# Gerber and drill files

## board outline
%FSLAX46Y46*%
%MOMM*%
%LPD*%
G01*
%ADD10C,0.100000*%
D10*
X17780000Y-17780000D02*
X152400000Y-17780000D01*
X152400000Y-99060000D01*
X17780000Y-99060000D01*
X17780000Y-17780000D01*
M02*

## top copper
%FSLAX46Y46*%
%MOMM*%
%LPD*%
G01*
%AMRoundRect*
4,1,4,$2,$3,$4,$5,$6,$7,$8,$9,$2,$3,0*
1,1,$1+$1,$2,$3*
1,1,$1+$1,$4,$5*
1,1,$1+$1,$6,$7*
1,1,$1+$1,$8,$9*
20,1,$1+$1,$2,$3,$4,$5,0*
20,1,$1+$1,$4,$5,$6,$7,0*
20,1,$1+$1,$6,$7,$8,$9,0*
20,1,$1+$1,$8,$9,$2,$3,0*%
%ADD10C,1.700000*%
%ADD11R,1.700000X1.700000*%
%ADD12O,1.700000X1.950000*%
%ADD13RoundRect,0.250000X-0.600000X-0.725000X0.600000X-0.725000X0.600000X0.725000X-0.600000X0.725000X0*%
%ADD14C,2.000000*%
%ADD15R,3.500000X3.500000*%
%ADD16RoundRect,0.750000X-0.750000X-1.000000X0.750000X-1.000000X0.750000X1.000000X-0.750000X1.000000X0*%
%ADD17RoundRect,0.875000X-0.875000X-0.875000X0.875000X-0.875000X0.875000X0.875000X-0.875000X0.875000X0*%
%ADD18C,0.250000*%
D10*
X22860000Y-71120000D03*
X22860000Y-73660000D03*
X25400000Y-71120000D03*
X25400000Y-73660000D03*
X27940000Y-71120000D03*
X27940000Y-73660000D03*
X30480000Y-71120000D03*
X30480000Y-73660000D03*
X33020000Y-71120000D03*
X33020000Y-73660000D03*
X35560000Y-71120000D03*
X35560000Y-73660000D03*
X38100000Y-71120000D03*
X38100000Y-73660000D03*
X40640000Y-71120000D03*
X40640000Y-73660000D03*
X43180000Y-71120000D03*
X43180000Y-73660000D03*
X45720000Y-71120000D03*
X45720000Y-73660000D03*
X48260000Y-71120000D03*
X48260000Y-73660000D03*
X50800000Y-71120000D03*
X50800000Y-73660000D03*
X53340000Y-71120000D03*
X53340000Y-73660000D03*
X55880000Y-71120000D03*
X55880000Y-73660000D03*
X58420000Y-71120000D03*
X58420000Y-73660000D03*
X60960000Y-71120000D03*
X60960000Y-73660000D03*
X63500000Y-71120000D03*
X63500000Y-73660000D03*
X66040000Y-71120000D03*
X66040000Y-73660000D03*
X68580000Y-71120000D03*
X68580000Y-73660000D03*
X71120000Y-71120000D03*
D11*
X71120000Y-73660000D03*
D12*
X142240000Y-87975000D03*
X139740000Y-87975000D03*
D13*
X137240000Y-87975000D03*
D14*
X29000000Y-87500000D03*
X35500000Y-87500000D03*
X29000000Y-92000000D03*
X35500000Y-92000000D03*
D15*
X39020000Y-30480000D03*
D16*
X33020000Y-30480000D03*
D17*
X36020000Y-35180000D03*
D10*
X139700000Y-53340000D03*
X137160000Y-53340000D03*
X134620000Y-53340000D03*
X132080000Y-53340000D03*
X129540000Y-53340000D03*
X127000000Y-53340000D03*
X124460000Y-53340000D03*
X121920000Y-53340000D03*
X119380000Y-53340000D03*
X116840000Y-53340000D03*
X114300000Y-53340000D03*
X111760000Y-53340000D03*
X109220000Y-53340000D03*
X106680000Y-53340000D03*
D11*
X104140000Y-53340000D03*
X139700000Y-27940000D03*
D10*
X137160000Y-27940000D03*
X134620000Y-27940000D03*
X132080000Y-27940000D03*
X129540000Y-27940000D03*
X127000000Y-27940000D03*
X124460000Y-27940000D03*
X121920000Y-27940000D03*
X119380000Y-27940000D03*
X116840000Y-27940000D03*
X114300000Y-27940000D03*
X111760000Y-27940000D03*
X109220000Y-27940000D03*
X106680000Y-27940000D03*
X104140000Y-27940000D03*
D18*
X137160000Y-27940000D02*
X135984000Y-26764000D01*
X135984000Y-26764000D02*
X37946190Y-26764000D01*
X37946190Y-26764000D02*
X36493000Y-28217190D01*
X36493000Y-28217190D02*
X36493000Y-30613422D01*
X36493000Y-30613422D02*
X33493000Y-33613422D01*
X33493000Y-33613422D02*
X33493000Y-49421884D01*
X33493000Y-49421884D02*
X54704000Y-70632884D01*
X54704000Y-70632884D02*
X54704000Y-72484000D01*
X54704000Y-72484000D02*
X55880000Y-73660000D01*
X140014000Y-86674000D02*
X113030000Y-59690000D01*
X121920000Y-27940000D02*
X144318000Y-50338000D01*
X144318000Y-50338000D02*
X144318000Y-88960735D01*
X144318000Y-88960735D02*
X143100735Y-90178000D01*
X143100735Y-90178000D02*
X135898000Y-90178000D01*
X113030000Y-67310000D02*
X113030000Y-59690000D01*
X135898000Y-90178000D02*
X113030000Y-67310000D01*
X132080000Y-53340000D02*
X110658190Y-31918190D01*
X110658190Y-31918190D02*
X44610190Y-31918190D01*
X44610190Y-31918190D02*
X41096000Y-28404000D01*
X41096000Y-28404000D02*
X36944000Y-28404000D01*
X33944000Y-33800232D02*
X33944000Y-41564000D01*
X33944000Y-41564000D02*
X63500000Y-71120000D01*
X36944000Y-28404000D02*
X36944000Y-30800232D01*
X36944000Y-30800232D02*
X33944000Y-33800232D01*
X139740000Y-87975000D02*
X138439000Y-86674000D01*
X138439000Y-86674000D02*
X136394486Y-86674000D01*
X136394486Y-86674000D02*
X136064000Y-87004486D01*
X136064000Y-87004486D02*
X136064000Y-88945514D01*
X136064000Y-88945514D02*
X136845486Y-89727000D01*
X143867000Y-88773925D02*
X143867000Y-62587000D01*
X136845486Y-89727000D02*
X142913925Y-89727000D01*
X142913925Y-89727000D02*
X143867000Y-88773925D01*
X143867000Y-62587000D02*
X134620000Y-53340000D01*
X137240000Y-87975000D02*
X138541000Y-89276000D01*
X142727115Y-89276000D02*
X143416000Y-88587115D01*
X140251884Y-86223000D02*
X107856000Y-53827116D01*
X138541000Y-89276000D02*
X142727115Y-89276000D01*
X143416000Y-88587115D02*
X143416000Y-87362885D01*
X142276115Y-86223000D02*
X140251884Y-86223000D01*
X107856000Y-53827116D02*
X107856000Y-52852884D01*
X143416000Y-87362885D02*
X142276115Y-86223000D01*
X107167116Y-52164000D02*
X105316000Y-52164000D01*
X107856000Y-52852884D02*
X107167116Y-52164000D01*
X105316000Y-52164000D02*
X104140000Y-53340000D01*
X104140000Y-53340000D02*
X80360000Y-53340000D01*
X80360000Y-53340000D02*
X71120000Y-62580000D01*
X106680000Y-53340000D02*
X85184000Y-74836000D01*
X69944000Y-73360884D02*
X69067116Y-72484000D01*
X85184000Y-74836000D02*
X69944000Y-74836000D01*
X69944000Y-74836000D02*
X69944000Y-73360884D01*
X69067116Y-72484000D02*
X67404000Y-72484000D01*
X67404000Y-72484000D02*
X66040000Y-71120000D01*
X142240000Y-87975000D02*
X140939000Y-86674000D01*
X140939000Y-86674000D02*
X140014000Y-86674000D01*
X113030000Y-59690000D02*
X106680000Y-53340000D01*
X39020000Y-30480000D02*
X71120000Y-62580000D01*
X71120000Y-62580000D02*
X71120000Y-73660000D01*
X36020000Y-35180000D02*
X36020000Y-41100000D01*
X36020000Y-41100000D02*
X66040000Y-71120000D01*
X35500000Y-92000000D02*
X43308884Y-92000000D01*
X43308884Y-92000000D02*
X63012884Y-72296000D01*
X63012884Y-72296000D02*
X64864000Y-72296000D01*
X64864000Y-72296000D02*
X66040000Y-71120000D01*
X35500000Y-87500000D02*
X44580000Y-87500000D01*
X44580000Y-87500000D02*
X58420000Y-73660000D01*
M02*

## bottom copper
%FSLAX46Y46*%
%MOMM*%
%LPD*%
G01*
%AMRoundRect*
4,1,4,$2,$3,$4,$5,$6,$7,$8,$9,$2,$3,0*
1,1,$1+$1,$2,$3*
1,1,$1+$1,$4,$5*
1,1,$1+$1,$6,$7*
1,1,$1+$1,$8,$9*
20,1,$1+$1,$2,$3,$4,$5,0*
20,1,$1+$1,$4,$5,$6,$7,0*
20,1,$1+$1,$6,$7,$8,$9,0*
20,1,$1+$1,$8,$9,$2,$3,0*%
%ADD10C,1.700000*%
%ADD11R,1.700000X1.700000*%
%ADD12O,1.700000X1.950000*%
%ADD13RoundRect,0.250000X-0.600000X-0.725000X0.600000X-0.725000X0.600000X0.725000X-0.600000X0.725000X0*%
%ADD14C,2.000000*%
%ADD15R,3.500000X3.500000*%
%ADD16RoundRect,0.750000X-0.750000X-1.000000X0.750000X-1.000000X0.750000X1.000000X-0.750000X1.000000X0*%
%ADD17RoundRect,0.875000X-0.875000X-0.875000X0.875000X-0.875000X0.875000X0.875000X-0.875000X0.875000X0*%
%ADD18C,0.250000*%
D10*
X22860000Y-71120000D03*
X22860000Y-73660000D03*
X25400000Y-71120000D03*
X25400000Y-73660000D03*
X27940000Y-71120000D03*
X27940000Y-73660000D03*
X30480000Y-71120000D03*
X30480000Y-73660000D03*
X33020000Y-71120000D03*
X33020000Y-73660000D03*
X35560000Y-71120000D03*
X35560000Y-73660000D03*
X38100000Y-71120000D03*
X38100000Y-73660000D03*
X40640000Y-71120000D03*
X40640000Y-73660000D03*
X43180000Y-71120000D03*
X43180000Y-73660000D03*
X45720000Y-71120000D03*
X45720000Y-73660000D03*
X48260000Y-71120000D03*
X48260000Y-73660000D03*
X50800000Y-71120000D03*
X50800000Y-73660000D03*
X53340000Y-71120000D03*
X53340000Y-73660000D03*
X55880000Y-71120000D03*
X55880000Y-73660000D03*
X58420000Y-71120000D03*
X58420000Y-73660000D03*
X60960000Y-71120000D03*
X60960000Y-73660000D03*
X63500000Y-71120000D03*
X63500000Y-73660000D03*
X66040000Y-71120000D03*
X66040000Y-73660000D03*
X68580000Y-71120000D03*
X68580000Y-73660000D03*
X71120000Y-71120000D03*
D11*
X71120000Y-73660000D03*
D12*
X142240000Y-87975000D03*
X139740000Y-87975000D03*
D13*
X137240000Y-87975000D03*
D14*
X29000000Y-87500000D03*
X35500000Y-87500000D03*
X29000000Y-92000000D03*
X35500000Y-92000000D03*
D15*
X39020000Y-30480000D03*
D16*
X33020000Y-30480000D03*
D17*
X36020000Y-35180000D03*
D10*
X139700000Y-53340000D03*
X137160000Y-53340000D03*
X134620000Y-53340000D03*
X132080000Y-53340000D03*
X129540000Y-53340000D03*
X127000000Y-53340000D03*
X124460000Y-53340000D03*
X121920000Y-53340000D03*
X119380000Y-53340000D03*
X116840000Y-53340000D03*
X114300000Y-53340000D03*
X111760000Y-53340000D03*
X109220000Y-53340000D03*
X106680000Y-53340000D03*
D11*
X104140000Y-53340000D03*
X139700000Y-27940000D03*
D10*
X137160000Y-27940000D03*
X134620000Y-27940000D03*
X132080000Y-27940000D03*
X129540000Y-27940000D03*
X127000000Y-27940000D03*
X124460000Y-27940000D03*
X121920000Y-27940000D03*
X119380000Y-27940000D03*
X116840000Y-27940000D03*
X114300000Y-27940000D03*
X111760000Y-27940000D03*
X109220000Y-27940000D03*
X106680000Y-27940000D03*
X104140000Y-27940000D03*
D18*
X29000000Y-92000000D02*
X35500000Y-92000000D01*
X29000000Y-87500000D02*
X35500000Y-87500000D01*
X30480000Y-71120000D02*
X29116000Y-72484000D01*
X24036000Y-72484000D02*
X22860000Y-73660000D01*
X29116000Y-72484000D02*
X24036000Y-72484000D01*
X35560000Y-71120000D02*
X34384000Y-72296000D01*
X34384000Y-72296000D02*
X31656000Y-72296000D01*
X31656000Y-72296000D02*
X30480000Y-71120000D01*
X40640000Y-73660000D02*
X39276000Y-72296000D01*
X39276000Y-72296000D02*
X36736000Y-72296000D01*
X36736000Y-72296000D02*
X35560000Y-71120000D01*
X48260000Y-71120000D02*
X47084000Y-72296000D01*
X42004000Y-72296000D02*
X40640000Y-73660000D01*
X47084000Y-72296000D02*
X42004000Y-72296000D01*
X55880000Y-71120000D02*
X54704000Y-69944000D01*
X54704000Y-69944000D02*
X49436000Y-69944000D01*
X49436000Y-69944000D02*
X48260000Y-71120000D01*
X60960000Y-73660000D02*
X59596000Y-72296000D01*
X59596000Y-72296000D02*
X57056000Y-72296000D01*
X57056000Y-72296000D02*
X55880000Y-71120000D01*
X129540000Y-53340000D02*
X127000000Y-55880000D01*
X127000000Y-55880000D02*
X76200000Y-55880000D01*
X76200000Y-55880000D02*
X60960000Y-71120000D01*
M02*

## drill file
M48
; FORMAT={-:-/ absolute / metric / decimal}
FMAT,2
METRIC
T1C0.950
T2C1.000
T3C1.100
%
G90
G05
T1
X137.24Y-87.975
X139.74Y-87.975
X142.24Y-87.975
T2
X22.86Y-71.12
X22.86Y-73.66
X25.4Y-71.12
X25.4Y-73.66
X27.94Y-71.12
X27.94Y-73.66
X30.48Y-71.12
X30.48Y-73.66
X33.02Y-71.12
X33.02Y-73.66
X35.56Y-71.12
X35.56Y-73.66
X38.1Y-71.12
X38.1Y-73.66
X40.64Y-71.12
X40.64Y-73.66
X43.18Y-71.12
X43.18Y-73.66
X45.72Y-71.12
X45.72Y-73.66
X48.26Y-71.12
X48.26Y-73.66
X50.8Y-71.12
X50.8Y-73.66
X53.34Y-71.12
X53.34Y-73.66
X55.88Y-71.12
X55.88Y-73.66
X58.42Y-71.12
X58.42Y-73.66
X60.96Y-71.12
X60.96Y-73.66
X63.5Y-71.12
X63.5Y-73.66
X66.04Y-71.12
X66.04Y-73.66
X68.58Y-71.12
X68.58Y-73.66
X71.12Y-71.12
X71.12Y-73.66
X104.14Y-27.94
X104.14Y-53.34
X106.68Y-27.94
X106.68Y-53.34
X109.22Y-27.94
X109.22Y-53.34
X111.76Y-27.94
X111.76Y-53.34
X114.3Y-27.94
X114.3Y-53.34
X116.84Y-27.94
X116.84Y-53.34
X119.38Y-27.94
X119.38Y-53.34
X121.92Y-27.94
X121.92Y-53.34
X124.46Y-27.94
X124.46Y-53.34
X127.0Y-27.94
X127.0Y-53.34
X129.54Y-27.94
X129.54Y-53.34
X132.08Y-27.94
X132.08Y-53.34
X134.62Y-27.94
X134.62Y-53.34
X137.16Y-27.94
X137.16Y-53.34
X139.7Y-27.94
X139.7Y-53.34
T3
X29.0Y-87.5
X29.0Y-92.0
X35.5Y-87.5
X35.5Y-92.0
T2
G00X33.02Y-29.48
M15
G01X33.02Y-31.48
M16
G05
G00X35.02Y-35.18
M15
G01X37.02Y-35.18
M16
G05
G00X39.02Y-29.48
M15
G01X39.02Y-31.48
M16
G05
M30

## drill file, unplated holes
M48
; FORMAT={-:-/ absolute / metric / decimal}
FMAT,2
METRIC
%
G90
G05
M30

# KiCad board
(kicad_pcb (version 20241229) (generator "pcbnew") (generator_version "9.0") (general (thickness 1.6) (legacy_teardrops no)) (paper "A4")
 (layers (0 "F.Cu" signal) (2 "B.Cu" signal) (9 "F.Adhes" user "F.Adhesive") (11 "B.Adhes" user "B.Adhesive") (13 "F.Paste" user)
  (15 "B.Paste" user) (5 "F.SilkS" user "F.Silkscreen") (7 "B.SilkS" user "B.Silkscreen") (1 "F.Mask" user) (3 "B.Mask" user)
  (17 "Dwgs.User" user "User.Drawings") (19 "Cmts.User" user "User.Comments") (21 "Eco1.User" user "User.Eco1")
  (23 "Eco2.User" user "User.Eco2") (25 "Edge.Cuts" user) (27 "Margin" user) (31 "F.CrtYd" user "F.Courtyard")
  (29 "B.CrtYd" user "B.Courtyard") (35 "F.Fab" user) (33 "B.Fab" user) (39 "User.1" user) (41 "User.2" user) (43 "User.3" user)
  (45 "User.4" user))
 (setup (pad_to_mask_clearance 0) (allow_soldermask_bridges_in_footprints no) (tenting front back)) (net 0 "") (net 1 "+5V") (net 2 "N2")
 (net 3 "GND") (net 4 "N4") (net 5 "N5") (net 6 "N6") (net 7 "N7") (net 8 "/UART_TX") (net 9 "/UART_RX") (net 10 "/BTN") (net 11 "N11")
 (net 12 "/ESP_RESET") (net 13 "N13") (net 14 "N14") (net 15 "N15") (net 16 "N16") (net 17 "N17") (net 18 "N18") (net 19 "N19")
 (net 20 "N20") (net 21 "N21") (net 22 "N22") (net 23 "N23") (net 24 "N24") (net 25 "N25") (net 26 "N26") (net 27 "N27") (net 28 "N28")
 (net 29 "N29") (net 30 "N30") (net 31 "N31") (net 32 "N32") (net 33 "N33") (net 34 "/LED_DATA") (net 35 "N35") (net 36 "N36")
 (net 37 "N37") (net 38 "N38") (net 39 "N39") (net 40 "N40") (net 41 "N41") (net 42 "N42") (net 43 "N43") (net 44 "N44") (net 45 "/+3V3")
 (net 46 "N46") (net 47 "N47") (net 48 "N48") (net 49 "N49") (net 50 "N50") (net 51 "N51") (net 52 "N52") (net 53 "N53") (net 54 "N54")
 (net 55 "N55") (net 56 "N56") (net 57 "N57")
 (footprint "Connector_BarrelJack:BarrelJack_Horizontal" (layer "F.Cu") (at 39.02 30.48)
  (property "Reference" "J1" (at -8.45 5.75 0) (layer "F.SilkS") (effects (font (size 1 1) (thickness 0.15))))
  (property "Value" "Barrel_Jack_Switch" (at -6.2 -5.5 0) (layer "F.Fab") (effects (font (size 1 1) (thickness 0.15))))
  (pad "1" thru_hole rect (at 0 0) (size 3.5 3.5) (drill oval 1 3) (layers "*.Cu" "*.Mask") (remove_unused_layers no) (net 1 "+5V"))
  (pad "2" thru_hole roundrect (at -6 0) (size 3 3.5) (drill oval 1 3) (layers "*.Cu" "*.Mask") (remove_unused_layers no)
   (roundrect_rratio 0.25) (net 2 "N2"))
  (pad "3" thru_hole roundrect (at -3 4.7) (size 3.5 3.5) (drill oval 3 1) (layers "*.Cu" "*.Mask") (remove_unused_layers no)
   (roundrect_rratio 0.25) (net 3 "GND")))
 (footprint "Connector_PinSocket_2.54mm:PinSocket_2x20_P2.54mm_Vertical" (layer "F.Cu") (at 71.12 73.66 -90)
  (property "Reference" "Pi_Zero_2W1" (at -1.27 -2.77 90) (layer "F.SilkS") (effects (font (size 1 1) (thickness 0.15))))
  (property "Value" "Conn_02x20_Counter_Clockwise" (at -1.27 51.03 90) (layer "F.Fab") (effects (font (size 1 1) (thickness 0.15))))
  (pad "1" thru_hole rect (at 0 0 270) (size 1.7 1.7) (drill 1) (layers "*.Cu" "*.Mask") (remove_unused_layers no) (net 1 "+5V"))
  (pad "2" thru_hole circle (at -2.54 0 270) (size 1.7 1.7) (drill 1) (layers "*.Cu" "*.Mask") (remove_unused_layers no) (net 1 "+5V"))
  (pad "3" thru_hole circle (at 0 2.54 270) (size 1.7 1.7) (drill 1) (layers "*.Cu" "*.Mask") (remove_unused_layers no) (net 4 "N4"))
  (pad "4" thru_hole circle (at -2.54 2.54 270) (size 1.7 1.7) (drill 1) (layers "*.Cu" "*.Mask") (remove_unused_layers no) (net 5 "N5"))
  (pad "5" thru_hole circle (at 0 5.08 270) (size 1.7 1.7) (drill 1) (layers "*.Cu" "*.Mask") (remove_unused_layers no) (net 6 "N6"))
  (pad "6" thru_hole circle (at -2.54 5.08 270) (size 1.7 1.7) (drill 1) (layers "*.Cu" "*.Mask") (remove_unused_layers no) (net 3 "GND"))
  (pad "7" thru_hole circle (at 0 7.62 270) (size 1.7 1.7) (drill 1) (layers "*.Cu" "*.Mask") (remove_unused_layers no) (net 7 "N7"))
  (pad "8" thru_hole circle (at -2.54 7.62 270) (size 1.7 1.7) (drill 1) (layers "*.Cu" "*.Mask") (remove_unused_layers no)
   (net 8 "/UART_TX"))
  (pad "9" thru_hole circle (at 0 10.16 270) (size 1.7 1.7) (drill 1) (layers "*.Cu" "*.Mask") (remove_unused_layers no) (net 3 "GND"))
  (pad "10" thru_hole circle (at -2.54 10.16 270) (size 1.7 1.7) (drill 1) (layers "*.Cu" "*.Mask") (remove_unused_layers no)
   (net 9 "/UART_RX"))
  (pad "11" thru_hole circle (at 0 12.7 270) (size 1.7 1.7) (drill 1) (layers "*.Cu" "*.Mask") (remove_unused_layers no) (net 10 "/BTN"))
  (pad "12" thru_hole circle (at -2.54 12.7 270) (size 1.7 1.7) (drill 1) (layers "*.Cu" "*.Mask") (remove_unused_layers no) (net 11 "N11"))
  (pad "13" thru_hole circle (at 0 15.24 270) (size 1.7 1.7) (drill 1) (layers "*.Cu" "*.Mask") (remove_unused_layers no)
   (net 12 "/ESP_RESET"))
  (pad "14" thru_hole circle (at -2.54 15.24 270) (size 1.7 1.7) (drill 1) (layers "*.Cu" "*.Mask") (remove_unused_layers no) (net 3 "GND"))
  (pad "15" thru_hole circle (at 0 17.78 270) (size 1.7 1.7) (drill 1) (layers "*.Cu" "*.Mask") (remove_unused_layers no) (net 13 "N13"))
  (pad "16" thru_hole circle (at -2.54 17.78 270) (size 1.7 1.7) (drill 1) (layers "*.Cu" "*.Mask") (remove_unused_layers no) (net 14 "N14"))
  (pad "17" thru_hole circle (at 0 20.32 270) (size 1.7 1.7) (drill 1) (layers "*.Cu" "*.Mask") (remove_unused_layers no) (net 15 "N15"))
  (pad "18" thru_hole circle (at -2.54 20.32 270) (size 1.7 1.7) (drill 1) (layers "*.Cu" "*.Mask") (remove_unused_layers no) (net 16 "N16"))
  (pad "19" thru_hole circle (at 0 22.86 270) (size 1.7 1.7) (drill 1) (layers "*.Cu" "*.Mask") (remove_unused_layers no) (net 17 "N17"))
  (pad "20" thru_hole circle (at -2.54 22.86 270) (size 1.7 1.7) (drill 1) (layers "*.Cu" "*.Mask") (remove_unused_layers no) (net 3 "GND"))
  (pad "21" thru_hole circle (at 0 25.4 270) (size 1.7 1.7) (drill 1) (layers "*.Cu" "*.Mask") (remove_unused_layers no) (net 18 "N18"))
  (pad "22" thru_hole circle (at -2.54 25.4 270) (size 1.7 1.7) (drill 1) (layers "*.Cu" "*.Mask") (remove_unused_layers no) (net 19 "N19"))
  (pad "23" thru_hole circle (at 0 27.94 270) (size 1.7 1.7) (drill 1) (layers "*.Cu" "*.Mask") (remove_unused_layers no) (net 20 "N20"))
  (pad "24" thru_hole circle (at -2.54 27.94 270) (size 1.7 1.7) (drill 1) (layers "*.Cu" "*.Mask") (remove_unused_layers no) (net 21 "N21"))
  (pad "25" thru_hole circle (at 0 30.48 270) (size 1.7 1.7) (drill 1) (layers "*.Cu" "*.Mask") (remove_unused_layers no) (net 3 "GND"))
  (pad "26" thru_hole circle (at -2.54 30.48 270) (size 1.7 1.7) (drill 1) (layers "*.Cu" "*.Mask") (remove_unused_layers no) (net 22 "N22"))
  (pad "27" thru_hole circle (at 0 33.02 270) (size 1.7 1.7) (drill 1) (layers "*.Cu" "*.Mask") (remove_unused_layers no) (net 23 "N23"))
  (pad "28" thru_hole circle (at -2.54 33.02 270) (size 1.7 1.7) (drill 1) (layers "*.Cu" "*.Mask") (remove_unused_layers no) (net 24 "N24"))
  (pad "29" thru_hole circle (at 0 35.56 270) (size 1.7 1.7) (drill 1) (layers "*.Cu" "*.Mask") (remove_unused_layers no) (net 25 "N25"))
  (pad "30" thru_hole circle (at -2.54 35.56 270) (size 1.7 1.7) (drill 1) (layers "*.Cu" "*.Mask") (remove_unused_layers no) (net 3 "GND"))
  (pad "31" thru_hole circle (at 0 38.1 270) (size 1.7 1.7) (drill 1) (layers "*.Cu" "*.Mask") (remove_unused_layers no) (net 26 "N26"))
  (pad "32" thru_hole circle (at -2.54 38.1 270) (size 1.7 1.7) (drill 1) (layers "*.Cu" "*.Mask") (remove_unused_layers no) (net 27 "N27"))
  (pad "33" thru_hole circle (at 0 40.64 270) (size 1.7 1.7) (drill 1) (layers "*.Cu" "*.Mask") (remove_unused_layers no) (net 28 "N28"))
  (pad "34" thru_hole circle (at -2.54 40.64 270) (size 1.7 1.7) (drill 1) (layers "*.Cu" "*.Mask") (remove_unused_layers no) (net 3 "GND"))
  (pad "35" thru_hole circle (at 0 43.18 270) (size 1.7 1.7) (drill 1) (layers "*.Cu" "*.Mask") (remove_unused_layers no) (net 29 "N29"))
  (pad "36" thru_hole circle (at -2.54 43.18 270) (size 1.7 1.7) (drill 1) (layers "*.Cu" "*.Mask") (remove_unused_layers no) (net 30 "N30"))
  (pad "37" thru_hole circle (at 0 45.72 270) (size 1.7 1.7) (drill 1) (layers "*.Cu" "*.Mask") (remove_unused_layers no) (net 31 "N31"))
  (pad "38" thru_hole circle (at -2.54 45.72 270) (size 1.7 1.7) (drill 1) (layers "*.Cu" "*.Mask") (remove_unused_layers no) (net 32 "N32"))
  (pad "39" thru_hole circle (at 0 48.26 270) (size 1.7 1.7) (drill 1) (layers "*.Cu" "*.Mask") (remove_unused_layers no) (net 3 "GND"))
  (pad "40" thru_hole circle (at -2.54 48.26 270) (size 1.7 1.7) (drill 1) (layers "*.Cu" "*.Mask") (remove_unused_layers no) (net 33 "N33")))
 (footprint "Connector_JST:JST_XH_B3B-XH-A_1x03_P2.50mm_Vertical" (layer "F.Cu") (at 137.24 87.975)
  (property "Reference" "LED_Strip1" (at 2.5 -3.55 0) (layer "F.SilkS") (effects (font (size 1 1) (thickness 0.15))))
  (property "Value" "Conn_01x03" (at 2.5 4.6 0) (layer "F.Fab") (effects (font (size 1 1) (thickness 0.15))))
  (pad "1" thru_hole roundrect (at 0 0) (size 1.7 1.95) (drill 0.95) (layers "*.Cu" "*.Mask") (remove_unused_layers no)
   (roundrect_rratio 0.147059) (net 1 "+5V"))
  (pad "2" thru_hole oval (at 2.5 0) (size 1.7 1.95) (drill 0.95) (layers "*.Cu" "*.Mask") (remove_unused_layers no) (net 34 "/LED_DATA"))
  (pad "3" thru_hole oval (at 5 0) (size 1.7 1.95) (drill 0.95) (layers "*.Cu" "*.Mask") (remove_unused_layers no) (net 3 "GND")))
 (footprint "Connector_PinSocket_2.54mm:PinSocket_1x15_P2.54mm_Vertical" (layer "F.Cu") (at 104.14 53.34 90)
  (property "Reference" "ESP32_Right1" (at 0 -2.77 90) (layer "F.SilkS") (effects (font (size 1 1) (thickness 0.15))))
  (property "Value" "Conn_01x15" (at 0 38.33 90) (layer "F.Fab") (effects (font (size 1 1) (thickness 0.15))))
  (pad "1" thru_hole rect (at 0 0 90) (size 1.7 1.7) (drill 1) (layers "*.Cu" "*.Mask") (remove_unused_layers no) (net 1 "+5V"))
  (pad "2" thru_hole circle (at 0 2.54 90) (size 1.7 1.7) (drill 1) (layers "*.Cu" "*.Mask") (remove_unused_layers no) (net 3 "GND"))
  (pad "3" thru_hole circle (at 0 5.08 90) (size 1.7 1.7) (drill 1) (layers "*.Cu" "*.Mask") (remove_unused_layers no) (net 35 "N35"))
  (pad "4" thru_hole circle (at 0 7.62 90) (size 1.7 1.7) (drill 1) (layers "*.Cu" "*.Mask") (remove_unused_layers no) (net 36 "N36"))
  (pad "5" thru_hole circle (at 0 10.16 90) (size 1.7 1.7) (drill 1) (layers "*.Cu" "*.Mask") (remove_unused_layers no) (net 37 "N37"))
  (pad "6" thru_hole circle (at 0 12.7 90) (size 1.7 1.7) (drill 1) (layers "*.Cu" "*.Mask") (remove_unused_layers no) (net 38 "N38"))
  (pad "7" thru_hole circle (at 0 15.24 90) (size 1.7 1.7) (drill 1) (layers "*.Cu" "*.Mask") (remove_unused_layers no) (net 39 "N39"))
  (pad "8" thru_hole circle (at 0 17.78 90) (size 1.7 1.7) (drill 1) (layers "*.Cu" "*.Mask") (remove_unused_layers no) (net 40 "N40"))
  (pad "9" thru_hole circle (at 0 20.32 90) (size 1.7 1.7) (drill 1) (layers "*.Cu" "*.Mask") (remove_unused_layers no) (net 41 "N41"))
  (pad "10" thru_hole circle (at 0 22.86 90) (size 1.7 1.7) (drill 1) (layers "*.Cu" "*.Mask") (remove_unused_layers no) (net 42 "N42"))
  (pad "11" thru_hole circle (at 0 25.4 90) (size 1.7 1.7) (drill 1) (layers "*.Cu" "*.Mask") (remove_unused_layers no) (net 9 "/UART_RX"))
  (pad "12" thru_hole circle (at 0 27.94 90) (size 1.7 1.7) (drill 1) (layers "*.Cu" "*.Mask") (remove_unused_layers no) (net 8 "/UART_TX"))
  (pad "13" thru_hole circle (at 0 30.48 90) (size 1.7 1.7) (drill 1) (layers "*.Cu" "*.Mask") (remove_unused_layers no)
   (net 34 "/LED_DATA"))
  (pad "14" thru_hole circle (at 0 33.02 90) (size 1.7 1.7) (drill 1) (layers "*.Cu" "*.Mask") (remove_unused_layers no) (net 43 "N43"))
  (pad "15" thru_hole circle (at 0 35.56 90) (size 1.7 1.7) (drill 1) (layers "*.Cu" "*.Mask") (remove_unused_layers no) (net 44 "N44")))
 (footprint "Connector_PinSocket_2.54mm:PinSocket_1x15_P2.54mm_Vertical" (layer "F.Cu") (at 139.7 27.94 -90)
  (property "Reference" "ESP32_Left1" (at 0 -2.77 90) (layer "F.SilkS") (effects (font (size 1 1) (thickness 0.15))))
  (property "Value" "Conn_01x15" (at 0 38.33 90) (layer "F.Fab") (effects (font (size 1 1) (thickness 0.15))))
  (pad "1" thru_hole rect (at 0 0 270) (size 1.7 1.7) (drill 1) (layers "*.Cu" "*.Mask") (remove_unused_layers no) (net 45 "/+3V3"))
  (pad "2" thru_hole circle (at 0 2.54 270) (size 1.7 1.7) (drill 1) (layers "*.Cu" "*.Mask") (remove_unused_layers no)
   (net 12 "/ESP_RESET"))
  (pad "3" thru_hole circle (at 0 5.08 270) (size 1.7 1.7) (drill 1) (layers "*.Cu" "*.Mask") (remove_unused_layers no) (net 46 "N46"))
  (pad "4" thru_hole circle (at 0 7.62 270) (size 1.7 1.7) (drill 1) (layers "*.Cu" "*.Mask") (remove_unused_layers no) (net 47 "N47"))
  (pad "5" thru_hole circle (at 0 10.16 270) (size 1.7 1.7) (drill 1) (layers "*.Cu" "*.Mask") (remove_unused_layers no) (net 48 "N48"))
  (pad "6" thru_hole circle (at 0 12.7 270) (size 1.7 1.7) (drill 1) (layers "*.Cu" "*.Mask") (remove_unused_layers no) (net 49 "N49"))
  (pad "7" thru_hole circle (at 0 15.24 270) (size 1.7 1.7) (drill 1) (layers "*.Cu" "*.Mask") (remove_unused_layers no) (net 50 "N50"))
  (pad "8" thru_hole circle (at 0 17.78 270) (size 1.7 1.7) (drill 1) (layers "*.Cu" "*.Mask") (remove_unused_layers no) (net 3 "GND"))
  (pad "9" thru_hole circle (at 0 20.32 270) (size 1.7 1.7) (drill 1) (layers "*.Cu" "*.Mask") (remove_unused_layers no) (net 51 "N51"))
  (pad "10" thru_hole circle (at 0 22.86 270) (size 1.7 1.7) (drill 1) (layers "*.Cu" "*.Mask") (remove_unused_layers no) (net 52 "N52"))
  (pad "11" thru_hole circle (at 0 25.4 270) (size 1.7 1.7) (drill 1) (layers "*.Cu" "*.Mask") (remove_unused_layers no) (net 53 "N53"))
  (pad "12" thru_hole circle (at 0 27.94 270) (size 1.7 1.7) (drill 1) (layers "*.Cu" "*.Mask") (remove_unused_layers no) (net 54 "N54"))
  (pad "13" thru_hole circle (at 0 30.48 270) (size 1.7 1.7) (drill 1) (layers "*.Cu" "*.Mask") (remove_unused_layers no) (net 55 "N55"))
  (pad "14" thru_hole circle (at 0 33.02 270) (size 1.7 1.7) (drill 1) (layers "*.Cu" "*.Mask") (remove_unused_layers no) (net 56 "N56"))
  (pad "15" thru_hole circle (at 0 35.56 270) (size 1.7 1.7) (drill 1) (layers "*.Cu" "*.Mask") (remove_unused_layers no) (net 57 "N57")))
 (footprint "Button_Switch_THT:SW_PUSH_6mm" (layer "F.Cu") (at 29 87.5)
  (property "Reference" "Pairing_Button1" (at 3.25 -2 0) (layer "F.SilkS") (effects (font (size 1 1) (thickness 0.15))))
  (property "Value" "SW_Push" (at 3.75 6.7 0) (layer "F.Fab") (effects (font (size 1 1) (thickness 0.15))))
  (pad "1" thru_hole circle (at 0 0 90) (size 2 2) (drill 1.1) (layers "*.Cu" "*.Mask") (remove_unused_layers no) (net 10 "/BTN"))
  (pad "1" thru_hole circle (at 6.5 0 90) (size 2 2) (drill 1.1) (layers "*.Cu" "*.Mask") (remove_unused_layers no) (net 10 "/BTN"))
  (pad "2" thru_hole circle (at 0 4.5 90) (size 2 2) (drill 1.1) (layers "*.Cu" "*.Mask") (remove_unused_layers no) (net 3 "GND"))
  (pad "2" thru_hole circle (at 6.5 4.5 90) (size 2 2) (drill 1.1) (layers "*.Cu" "*.Mask") (remove_unused_layers no) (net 3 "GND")))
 (gr_rect (start 17.78 17.78) (end 152.4 99.06) (stroke (width 0.1) (type default)) (fill no) (layer "Edge.Cuts"))
 (segment (start 54.704 70.632884) (end 54.704 72.484) (width 0.25) (layer "F.Cu") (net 12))
 (segment (start 36.493 30.613422) (end 33.493 33.613422) (width 0.25) (layer "F.Cu") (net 12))
 (segment (start 37.94619 26.764) (end 36.493 28.21719) (width 0.25) (layer "F.Cu") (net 12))
 (segment (start 137.16 27.94) (end 135.984 26.764) (width 0.25) (layer "F.Cu") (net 12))
 (segment (start 36.493 28.21719) (end 36.493 30.613422) (width 0.25) (layer "F.Cu") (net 12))
 (segment (start 33.493 49.421884) (end 54.704 70.632884) (width 0.25) (layer "F.Cu") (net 12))
 (segment (start 33.493 33.613422) (end 33.493 49.421884) (width 0.25) (layer "F.Cu") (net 12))
 (segment (start 54.704 72.484) (end 55.88 73.66) (width 0.25) (layer "F.Cu") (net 12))
 (segment (start 135.984 26.764) (end 37.94619 26.764) (width 0.25) (layer "F.Cu") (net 12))
 (segment (start 36.02 35.18) (end 36.02 41.1) (width 0.25) (layer "F.Cu") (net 3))
 (segment (start 43.308884 92) (end 63.012884 72.296) (width 0.25) (layer "F.Cu") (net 3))
 (segment (start 85.184 74.836) (end 69.944 74.836) (width 0.25) (layer "F.Cu") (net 3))
 (segment (start 113.03 67.31) (end 113.03 59.69) (width 0.25) (layer "F.Cu") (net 3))
 (segment (start 142.24 87.975) (end 140.939 86.674) (width 0.25) (layer "F.Cu") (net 3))
 (segment (start 144.318 50.338) (end 144.318 88.960735) (width 0.25) (layer "F.Cu") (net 3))
 (segment (start 35.5 92) (end 43.308884 92) (width 0.25) (layer "F.Cu") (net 3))
 (segment (start 135.898 90.178) (end 113.03 67.31) (width 0.25) (layer "F.Cu") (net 3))
 (segment (start 69.944 74.836) (end 69.944 73.360884) (width 0.25) (layer "F.Cu") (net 3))
 (segment (start 140.014 86.674) (end 113.03 59.69) (width 0.25) (layer "F.Cu") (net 3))
 (segment (start 144.318 88.960735) (end 143.100735 90.178) (width 0.25) (layer "F.Cu") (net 3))
 (segment (start 63.012884 72.296) (end 64.864 72.296) (width 0.25) (layer "F.Cu") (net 3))
 (segment (start 143.100735 90.178) (end 135.898 90.178) (width 0.25) (layer "F.Cu") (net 3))
 (segment (start 67.404 72.484) (end 66.04 71.12) (width 0.25) (layer "F.Cu") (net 3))
 (segment (start 113.03 59.69) (end 106.68 53.34) (width 0.25) (layer "F.Cu") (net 3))
 (segment (start 106.68 53.34) (end 85.184 74.836) (width 0.25) (layer "F.Cu") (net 3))
 (segment (start 140.939 86.674) (end 140.014 86.674) (width 0.25) (layer "F.Cu") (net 3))
 (segment (start 69.067116 72.484) (end 67.404 72.484) (width 0.25) (layer "F.Cu") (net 3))
 (segment (start 121.92 27.94) (end 144.318 50.338) (width 0.25) (layer "F.Cu") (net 3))
 (segment (start 36.02 41.1) (end 66.04 71.12) (width 0.25) (layer "F.Cu") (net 3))
 (segment (start 64.864 72.296) (end 66.04 71.12) (width 0.25) (layer "F.Cu") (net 3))
 (segment (start 69.944 73.360884) (end 69.067116 72.484) (width 0.25) (layer "F.Cu") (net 3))
 (segment (start 31.656 72.296) (end 30.48 71.12) (width 0.25) (layer "B.Cu") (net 3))
 (segment (start 24.036 72.484) (end 22.86 73.66) (width 0.25) (layer "B.Cu") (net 3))
 (segment (start 29.116 72.484) (end 24.036 72.484) (width 0.25) (layer "B.Cu") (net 3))
 (segment (start 34.384 72.296) (end 31.656 72.296) (width 0.25) (layer "B.Cu") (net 3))
 (segment (start 60.96 73.66) (end 59.596 72.296) (width 0.25) (layer "B.Cu") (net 3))
 (segment (start 36.736 72.296) (end 35.56 71.12) (width 0.25) (layer "B.Cu") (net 3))
 (segment (start 54.704 69.944) (end 49.436 69.944) (width 0.25) (layer "B.Cu") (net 3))
 (segment (start 49.436 69.944) (end 48.26 71.12) (width 0.25) (layer "B.Cu") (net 3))
 (segment (start 57.056 72.296) (end 55.88 71.12) (width 0.25) (layer "B.Cu") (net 3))
 (segment (start 35.56 71.12) (end 34.384 72.296) (width 0.25) (layer "B.Cu") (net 3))
 (segment (start 30.48 71.12) (end 29.116 72.484) (width 0.25) (layer "B.Cu") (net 3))
 (segment (start 40.64 73.66) (end 39.276 72.296) (width 0.25) (layer "B.Cu") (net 3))
 (segment (start 59.596 72.296) (end 57.056 72.296) (width 0.25) (layer "B.Cu") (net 3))
 (segment (start 48.26 71.12) (end 47.084 72.296) (width 0.25) (layer "B.Cu") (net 3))
 (segment (start 55.88 71.12) (end 54.704 69.944) (width 0.25) (layer "B.Cu") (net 3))
 (segment (start 42.004 72.296) (end 40.64 73.66) (width 0.25) (layer "B.Cu") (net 3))
 (segment (start 29 92) (end 35.5 92) (width 0.25) (layer "B.Cu") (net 3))
 (segment (start 39.276 72.296) (end 36.736 72.296) (width 0.25) (layer "B.Cu") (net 3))
 (segment (start 47.084 72.296) (end 42.004 72.296) (width 0.25) (layer "B.Cu") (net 3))
 (segment (start 36.944 28.404) (end 36.944 30.800232) (width 0.25) (layer "F.Cu") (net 8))
 (segment (start 33.944 41.564) (end 63.5 71.12) (width 0.25) (layer "F.Cu") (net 8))
 (segment (start 132.08 53.34) (end 110.65819 31.91819) (width 0.25) (layer "F.Cu") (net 8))
 (segment (start 44.61019 31.91819) (end 41.096 28.404) (width 0.25) (layer "F.Cu") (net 8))
 (segment (start 110.65819 31.91819) (end 44.61019 31.91819) (width 0.25) (layer "F.Cu") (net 8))
 (segment (start 41.096 28.404) (end 36.944 28.404) (width 0.25) (layer "F.Cu") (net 8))
 (segment (start 36.944 30.800232) (end 33.944 33.800232) (width 0.25) (layer "F.Cu") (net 8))
 (segment (start 33.944 33.800232) (end 33.944 41.564) (width 0.25) (layer "F.Cu") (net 8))
 (segment (start 127 55.88) (end 76.2 55.88) (width 0.25) (layer "B.Cu") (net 9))
 (segment (start 129.54 53.34) (end 127 55.88) (width 0.25) (layer "B.Cu") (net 9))
 (segment (start 76.2 55.88) (end 60.96 71.12) (width 0.25) (layer "B.Cu") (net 9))
 (segment (start 142.913925 89.727) (end 143.867 88.773925) (width 0.25) (layer "F.Cu") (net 34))
 (segment (start 138.439 86.674) (end 136.394486 86.674) (width 0.25) (layer "F.Cu") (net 34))
 (segment (start 136.845486 89.727) (end 142.913925 89.727) (width 0.25) (layer "F.Cu") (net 34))
 (segment (start 136.394486 86.674) (end 136.064 87.004486) (width 0.25) (layer "F.Cu") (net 34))
 (segment (start 139.74 87.975) (end 138.439 86.674) (width 0.25) (layer "F.Cu") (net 34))
 (segment (start 136.064 88.945514) (end 136.845486 89.727) (width 0.25) (layer "F.Cu") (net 34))
 (segment (start 143.867 88.773925) (end 143.867 62.587) (width 0.25) (layer "F.Cu") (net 34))
 (segment (start 143.867 62.587) (end 134.62 53.34) (width 0.25) (layer "F.Cu") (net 34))
 (segment (start 136.064 87.004486) (end 136.064 88.945514) (width 0.25) (layer "F.Cu") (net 34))
 (segment (start 80.36 53.34) (end 71.12 62.58) (width 0.25) (layer "F.Cu") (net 1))
 (segment (start 39.02 30.48) (end 71.12 62.58) (width 0.25) (layer "F.Cu") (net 1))
 (segment (start 138.541 89.276) (end 142.727115 89.276) (width 0.25) (layer "F.Cu") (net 1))
 (segment (start 142.276115 86.223) (end 140.251884 86.223) (width 0.25) (layer "F.Cu") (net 1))
 (segment (start 137.24 87.975) (end 138.541 89.276) (width 0.25) (layer "F.Cu") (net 1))
 (segment (start 107.856 52.852884) (end 107.167116 52.164) (width 0.25) (layer "F.Cu") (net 1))
 (segment (start 143.416 87.362885) (end 142.276115 86.223) (width 0.25) (layer "F.Cu") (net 1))
 (segment (start 71.12 62.58) (end 71.12 73.66) (width 0.25) (layer "F.Cu") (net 1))
 (segment (start 105.316 52.164) (end 104.14 53.34) (width 0.25) (layer "F.Cu") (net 1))
 (segment (start 104.14 53.34) (end 80.36 53.34) (width 0.25) (layer "F.Cu") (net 1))
 (segment (start 107.856 53.827116) (end 107.856 52.852884) (width 0.25) (layer "F.Cu") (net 1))
 (segment (start 142.727115 89.276) (end 143.416 88.587115) (width 0.25) (layer "F.Cu") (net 1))
 (segment (start 107.167116 52.164) (end 105.316 52.164) (width 0.25) (layer "F.Cu") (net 1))
 (segment (start 143.416 88.587115) (end 143.416 87.362885) (width 0.25) (layer "F.Cu") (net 1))
 (segment (start 140.251884 86.223) (end 107.856 53.827116) (width 0.25) (layer "F.Cu") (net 1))
 (segment (start 35.5 87.5) (end 44.58 87.5) (width 0.25) (layer "F.Cu") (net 10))
 (segment (start 44.58 87.5) (end 58.42 73.66) (width 0.25) (layer "F.Cu") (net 10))
 (segment (start 29 87.5) (end 35.5 87.5) (width 0.25) (layer "B.Cu") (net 10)))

